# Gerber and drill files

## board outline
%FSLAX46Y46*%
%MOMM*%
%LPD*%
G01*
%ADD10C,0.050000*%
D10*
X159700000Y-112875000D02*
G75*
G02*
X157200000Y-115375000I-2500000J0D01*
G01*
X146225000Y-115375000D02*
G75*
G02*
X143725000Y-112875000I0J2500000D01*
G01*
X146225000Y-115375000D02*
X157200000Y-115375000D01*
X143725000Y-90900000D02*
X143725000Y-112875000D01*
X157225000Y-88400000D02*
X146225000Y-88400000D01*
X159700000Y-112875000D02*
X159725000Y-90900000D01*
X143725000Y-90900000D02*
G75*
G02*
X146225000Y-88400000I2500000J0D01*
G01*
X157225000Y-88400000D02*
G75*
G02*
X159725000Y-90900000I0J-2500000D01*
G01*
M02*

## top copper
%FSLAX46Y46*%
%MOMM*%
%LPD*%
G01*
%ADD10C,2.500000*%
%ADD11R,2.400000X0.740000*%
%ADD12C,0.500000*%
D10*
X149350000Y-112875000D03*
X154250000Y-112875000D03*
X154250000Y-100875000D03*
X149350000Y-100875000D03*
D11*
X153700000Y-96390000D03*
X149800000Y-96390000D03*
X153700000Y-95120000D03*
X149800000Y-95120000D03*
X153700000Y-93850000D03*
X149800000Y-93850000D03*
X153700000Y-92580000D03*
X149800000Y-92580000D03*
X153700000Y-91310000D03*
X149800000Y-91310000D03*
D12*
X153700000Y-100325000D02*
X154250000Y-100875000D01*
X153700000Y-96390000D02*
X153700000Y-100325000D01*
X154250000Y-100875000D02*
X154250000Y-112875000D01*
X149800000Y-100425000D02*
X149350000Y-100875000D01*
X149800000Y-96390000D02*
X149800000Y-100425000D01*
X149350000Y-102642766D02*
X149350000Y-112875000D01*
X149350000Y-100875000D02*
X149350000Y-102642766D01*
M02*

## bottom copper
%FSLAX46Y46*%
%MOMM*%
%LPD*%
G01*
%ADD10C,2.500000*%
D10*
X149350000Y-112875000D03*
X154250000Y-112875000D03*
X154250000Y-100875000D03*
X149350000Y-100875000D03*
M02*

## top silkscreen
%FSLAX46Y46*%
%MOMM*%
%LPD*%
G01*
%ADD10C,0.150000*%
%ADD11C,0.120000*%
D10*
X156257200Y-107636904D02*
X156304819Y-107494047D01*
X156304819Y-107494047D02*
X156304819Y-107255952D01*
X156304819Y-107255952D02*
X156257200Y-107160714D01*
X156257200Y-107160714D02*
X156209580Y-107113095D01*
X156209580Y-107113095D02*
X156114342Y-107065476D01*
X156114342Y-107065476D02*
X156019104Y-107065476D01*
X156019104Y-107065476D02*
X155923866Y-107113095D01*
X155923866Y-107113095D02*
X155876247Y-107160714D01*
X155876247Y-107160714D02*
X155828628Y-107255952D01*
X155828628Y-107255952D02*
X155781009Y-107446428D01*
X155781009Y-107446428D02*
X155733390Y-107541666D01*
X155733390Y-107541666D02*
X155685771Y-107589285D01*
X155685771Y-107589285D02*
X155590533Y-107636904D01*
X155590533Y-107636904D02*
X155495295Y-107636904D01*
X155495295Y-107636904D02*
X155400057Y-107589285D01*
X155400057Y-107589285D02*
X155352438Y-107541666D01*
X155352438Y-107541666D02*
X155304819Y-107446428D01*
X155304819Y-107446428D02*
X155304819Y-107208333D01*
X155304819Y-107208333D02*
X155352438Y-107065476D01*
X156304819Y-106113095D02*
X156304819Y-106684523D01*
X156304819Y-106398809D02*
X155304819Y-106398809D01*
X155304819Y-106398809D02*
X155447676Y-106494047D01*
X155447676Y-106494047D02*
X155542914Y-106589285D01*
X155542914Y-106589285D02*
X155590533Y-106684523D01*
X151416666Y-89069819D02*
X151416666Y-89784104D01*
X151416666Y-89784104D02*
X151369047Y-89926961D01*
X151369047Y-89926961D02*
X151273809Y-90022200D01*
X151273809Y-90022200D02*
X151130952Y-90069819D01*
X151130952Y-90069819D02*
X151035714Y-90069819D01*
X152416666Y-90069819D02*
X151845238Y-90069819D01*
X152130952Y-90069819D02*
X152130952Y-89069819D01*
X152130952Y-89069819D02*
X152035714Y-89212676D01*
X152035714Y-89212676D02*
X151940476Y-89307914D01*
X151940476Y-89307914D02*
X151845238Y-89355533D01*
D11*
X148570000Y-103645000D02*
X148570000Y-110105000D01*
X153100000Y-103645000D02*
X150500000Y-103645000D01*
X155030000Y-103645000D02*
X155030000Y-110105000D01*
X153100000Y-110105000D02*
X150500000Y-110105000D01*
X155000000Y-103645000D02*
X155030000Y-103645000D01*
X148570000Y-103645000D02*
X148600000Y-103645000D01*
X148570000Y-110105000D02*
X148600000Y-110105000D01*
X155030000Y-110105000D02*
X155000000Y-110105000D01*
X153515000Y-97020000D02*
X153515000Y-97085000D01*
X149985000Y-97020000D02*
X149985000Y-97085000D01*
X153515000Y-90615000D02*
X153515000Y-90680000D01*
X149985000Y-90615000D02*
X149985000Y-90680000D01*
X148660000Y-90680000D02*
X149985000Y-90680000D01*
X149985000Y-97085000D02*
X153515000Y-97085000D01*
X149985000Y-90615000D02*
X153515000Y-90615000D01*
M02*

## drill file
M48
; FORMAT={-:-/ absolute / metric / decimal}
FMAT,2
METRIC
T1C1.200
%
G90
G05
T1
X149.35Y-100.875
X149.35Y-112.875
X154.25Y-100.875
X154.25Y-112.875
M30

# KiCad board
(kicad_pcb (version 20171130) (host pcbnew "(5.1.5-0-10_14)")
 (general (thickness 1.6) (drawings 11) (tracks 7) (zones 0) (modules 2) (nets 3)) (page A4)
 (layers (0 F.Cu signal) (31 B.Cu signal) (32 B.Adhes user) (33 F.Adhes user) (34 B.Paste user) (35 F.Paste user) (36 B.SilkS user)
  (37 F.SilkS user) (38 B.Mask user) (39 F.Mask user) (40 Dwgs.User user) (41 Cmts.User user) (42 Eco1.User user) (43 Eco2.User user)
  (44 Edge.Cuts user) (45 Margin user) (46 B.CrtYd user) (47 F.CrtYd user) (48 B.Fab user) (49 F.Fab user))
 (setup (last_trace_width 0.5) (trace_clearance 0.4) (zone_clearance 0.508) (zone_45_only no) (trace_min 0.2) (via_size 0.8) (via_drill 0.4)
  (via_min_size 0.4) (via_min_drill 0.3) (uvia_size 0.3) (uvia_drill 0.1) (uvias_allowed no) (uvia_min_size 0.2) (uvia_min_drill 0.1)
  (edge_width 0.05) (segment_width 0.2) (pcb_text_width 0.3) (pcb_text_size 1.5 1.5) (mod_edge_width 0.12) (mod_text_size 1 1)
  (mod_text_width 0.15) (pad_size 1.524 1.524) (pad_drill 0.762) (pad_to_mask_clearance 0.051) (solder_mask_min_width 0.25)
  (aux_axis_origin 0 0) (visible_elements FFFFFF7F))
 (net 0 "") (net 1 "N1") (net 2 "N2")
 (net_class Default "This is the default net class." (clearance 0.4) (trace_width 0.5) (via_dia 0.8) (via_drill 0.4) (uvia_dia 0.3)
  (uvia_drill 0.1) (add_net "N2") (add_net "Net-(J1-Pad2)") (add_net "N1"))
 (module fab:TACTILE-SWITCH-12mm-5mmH (layer F.Cu) (at 151.8 106.875 270)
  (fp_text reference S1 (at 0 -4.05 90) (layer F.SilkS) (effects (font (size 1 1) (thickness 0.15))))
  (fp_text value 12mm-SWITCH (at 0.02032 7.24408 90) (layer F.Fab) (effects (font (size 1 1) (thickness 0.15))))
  (fp_line (start -3.23 3.23) (end 3.23 3.23) (layer F.SilkS) (width 0.12))
  (fp_line (start -3.23 -1.3) (end -3.23 1.3) (layer F.SilkS) (width 0.12))
  (fp_line (start -3.23 -3.23) (end 3.23 -3.23) (layer F.SilkS) (width 0.12))
  (fp_line (start 3.23 -1.3) (end 3.23 1.3) (layer F.SilkS) (width 0.12))
  (fp_line (start -3.23 -3.2) (end -3.23 -3.23) (layer F.SilkS) (width 0.12))
  (fp_line (start -3.23 3.23) (end -3.23 3.2) (layer F.SilkS) (width 0.12))
  (fp_line (start 3.23 3.23) (end 3.23 3.2) (layer F.SilkS) (width 0.12))
  (fp_line (start 3.23 -3.23) (end 3.23 -3.2) (layer F.SilkS) (width 0.12))
  (pad 4 thru_hole circle (at 6 2.45 270) (size 2.5 2.5) (drill 1.2) (layers *.Cu *.Mask) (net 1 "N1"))
  (pad 2 thru_hole circle (at 6 -2.45 270) (size 2.5 2.5) (drill 1.2) (layers *.Cu *.Mask) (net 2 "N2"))
  (pad 1 thru_hole circle (at -6 -2.45 270) (size 2.5 2.5) (drill 1.2) (layers *.Cu *.Mask) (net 2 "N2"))
  (pad 3 thru_hole circle (at -6 2.45 270) (size 2.5 2.5) (drill 1.2) (layers *.Cu *.Mask) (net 1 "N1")))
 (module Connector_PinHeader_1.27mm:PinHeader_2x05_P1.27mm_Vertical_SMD (layer F.Cu) (at 151.75 93.85)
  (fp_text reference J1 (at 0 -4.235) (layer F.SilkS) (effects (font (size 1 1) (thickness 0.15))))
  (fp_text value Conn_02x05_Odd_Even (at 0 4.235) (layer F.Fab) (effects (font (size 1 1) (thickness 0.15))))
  (fp_line (start 1.765 3.17) (end 1.765 3.235) (layer F.SilkS) (width 0.12))
  (fp_line (start -1.765 3.17) (end -1.765 3.235) (layer F.SilkS) (width 0.12))
  (fp_line (start 1.765 -3.235) (end 1.765 -3.17) (layer F.SilkS) (width 0.12))
  (fp_line (start -1.765 -3.235) (end -1.765 -3.17) (layer F.SilkS) (width 0.12))
  (fp_line (start -3.09 -3.17) (end -1.765 -3.17) (layer F.SilkS) (width 0.12))
  (fp_line (start -1.765 3.235) (end 1.765 3.235) (layer F.SilkS) (width 0.12))
  (fp_line (start -1.765 -3.235) (end 1.765 -3.235) (layer F.SilkS) (width 0.12))
  (pad 10 smd rect (at 1.95 2.54) (size 2.4 0.74) (layers F.Cu F.Paste F.Mask) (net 2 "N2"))
  (pad 9 smd rect (at -1.95 2.54) (size 2.4 0.74) (layers F.Cu F.Paste F.Mask) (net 1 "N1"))
  (pad 8 smd rect (at 1.95 1.27) (size 2.4 0.74) (layers F.Cu F.Paste F.Mask))
  (pad 7 smd rect (at -1.95 1.27) (size 2.4 0.74) (layers F.Cu F.Paste F.Mask))
  (pad 6 smd rect (at 1.95 0) (size 2.4 0.74) (layers F.Cu F.Paste F.Mask))
  (pad 5 smd rect (at -1.95 0) (size 2.4 0.74) (layers F.Cu F.Paste F.Mask))
  (pad 4 smd rect (at 1.95 -1.27) (size 2.4 0.74) (layers F.Cu F.Paste F.Mask))
  (pad 3 smd rect (at -1.95 -1.27) (size 2.4 0.74) (layers F.Cu F.Paste F.Mask))
  (pad 2 smd rect (at 1.95 -2.54) (size 2.4 0.74) (layers F.Cu F.Paste F.Mask))
  (pad 1 smd rect (at -1.95 -2.54) (size 2.4 0.74) (layers F.Cu F.Paste F.Mask)))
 (gr_arc (start 157.2 112.875) (end 157.2 115.375) (angle -90) (layer Edge.Cuts) (width 0.05))
 (gr_arc (start 146.225 112.875) (end 143.725 112.875) (angle -90) (layer Edge.Cuts) (width 0.05))
 (gr_line (start 146.225 115.375) (end 157.2 115.375) (layer Edge.Cuts) (width 0.05))
 (gr_line (start 143.725 90.9) (end 143.725 112.875) (layer Edge.Cuts) (width 0.05))
 (gr_line (start 157.225 88.4) (end 146.225 88.4) (layer Edge.Cuts) (width 0.05))
 (gr_line (start 159.7 112.875) (end 159.725 90.9) (layer Edge.Cuts) (width 0.05))
 (gr_arc (start 146.225 90.9) (end 146.225 88.4) (angle -90) (layer Edge.Cuts) (width 0.05))
 (gr_arc (start 157.225 90.9) (end 159.725 90.9) (angle -90) (layer Edge.Cuts) (width 0.05))
 (segment (start 153.7 100.325) (end 154.25 100.875) (width 0.5) (layer F.Cu) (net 2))
 (segment (start 153.7 96.39) (end 153.7 100.325) (width 0.5) (layer F.Cu) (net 2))
 (segment (start 154.25 100.875) (end 154.25 112.875) (width 0.5) (layer F.Cu) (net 2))
 (segment (start 149.8 100.425) (end 149.35 100.875) (width 0.5) (layer F.Cu) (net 1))
 (segment (start 149.8 96.39) (end 149.8 100.425) (width 0.5) (layer F.Cu) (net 1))
 (segment (start 149.35 102.642766) (end 149.35 112.875) (width 0.5) (layer F.Cu) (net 1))
 (segment (start 149.35 100.875) (end 149.35 102.642766) (width 0.5) (layer F.Cu) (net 1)))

